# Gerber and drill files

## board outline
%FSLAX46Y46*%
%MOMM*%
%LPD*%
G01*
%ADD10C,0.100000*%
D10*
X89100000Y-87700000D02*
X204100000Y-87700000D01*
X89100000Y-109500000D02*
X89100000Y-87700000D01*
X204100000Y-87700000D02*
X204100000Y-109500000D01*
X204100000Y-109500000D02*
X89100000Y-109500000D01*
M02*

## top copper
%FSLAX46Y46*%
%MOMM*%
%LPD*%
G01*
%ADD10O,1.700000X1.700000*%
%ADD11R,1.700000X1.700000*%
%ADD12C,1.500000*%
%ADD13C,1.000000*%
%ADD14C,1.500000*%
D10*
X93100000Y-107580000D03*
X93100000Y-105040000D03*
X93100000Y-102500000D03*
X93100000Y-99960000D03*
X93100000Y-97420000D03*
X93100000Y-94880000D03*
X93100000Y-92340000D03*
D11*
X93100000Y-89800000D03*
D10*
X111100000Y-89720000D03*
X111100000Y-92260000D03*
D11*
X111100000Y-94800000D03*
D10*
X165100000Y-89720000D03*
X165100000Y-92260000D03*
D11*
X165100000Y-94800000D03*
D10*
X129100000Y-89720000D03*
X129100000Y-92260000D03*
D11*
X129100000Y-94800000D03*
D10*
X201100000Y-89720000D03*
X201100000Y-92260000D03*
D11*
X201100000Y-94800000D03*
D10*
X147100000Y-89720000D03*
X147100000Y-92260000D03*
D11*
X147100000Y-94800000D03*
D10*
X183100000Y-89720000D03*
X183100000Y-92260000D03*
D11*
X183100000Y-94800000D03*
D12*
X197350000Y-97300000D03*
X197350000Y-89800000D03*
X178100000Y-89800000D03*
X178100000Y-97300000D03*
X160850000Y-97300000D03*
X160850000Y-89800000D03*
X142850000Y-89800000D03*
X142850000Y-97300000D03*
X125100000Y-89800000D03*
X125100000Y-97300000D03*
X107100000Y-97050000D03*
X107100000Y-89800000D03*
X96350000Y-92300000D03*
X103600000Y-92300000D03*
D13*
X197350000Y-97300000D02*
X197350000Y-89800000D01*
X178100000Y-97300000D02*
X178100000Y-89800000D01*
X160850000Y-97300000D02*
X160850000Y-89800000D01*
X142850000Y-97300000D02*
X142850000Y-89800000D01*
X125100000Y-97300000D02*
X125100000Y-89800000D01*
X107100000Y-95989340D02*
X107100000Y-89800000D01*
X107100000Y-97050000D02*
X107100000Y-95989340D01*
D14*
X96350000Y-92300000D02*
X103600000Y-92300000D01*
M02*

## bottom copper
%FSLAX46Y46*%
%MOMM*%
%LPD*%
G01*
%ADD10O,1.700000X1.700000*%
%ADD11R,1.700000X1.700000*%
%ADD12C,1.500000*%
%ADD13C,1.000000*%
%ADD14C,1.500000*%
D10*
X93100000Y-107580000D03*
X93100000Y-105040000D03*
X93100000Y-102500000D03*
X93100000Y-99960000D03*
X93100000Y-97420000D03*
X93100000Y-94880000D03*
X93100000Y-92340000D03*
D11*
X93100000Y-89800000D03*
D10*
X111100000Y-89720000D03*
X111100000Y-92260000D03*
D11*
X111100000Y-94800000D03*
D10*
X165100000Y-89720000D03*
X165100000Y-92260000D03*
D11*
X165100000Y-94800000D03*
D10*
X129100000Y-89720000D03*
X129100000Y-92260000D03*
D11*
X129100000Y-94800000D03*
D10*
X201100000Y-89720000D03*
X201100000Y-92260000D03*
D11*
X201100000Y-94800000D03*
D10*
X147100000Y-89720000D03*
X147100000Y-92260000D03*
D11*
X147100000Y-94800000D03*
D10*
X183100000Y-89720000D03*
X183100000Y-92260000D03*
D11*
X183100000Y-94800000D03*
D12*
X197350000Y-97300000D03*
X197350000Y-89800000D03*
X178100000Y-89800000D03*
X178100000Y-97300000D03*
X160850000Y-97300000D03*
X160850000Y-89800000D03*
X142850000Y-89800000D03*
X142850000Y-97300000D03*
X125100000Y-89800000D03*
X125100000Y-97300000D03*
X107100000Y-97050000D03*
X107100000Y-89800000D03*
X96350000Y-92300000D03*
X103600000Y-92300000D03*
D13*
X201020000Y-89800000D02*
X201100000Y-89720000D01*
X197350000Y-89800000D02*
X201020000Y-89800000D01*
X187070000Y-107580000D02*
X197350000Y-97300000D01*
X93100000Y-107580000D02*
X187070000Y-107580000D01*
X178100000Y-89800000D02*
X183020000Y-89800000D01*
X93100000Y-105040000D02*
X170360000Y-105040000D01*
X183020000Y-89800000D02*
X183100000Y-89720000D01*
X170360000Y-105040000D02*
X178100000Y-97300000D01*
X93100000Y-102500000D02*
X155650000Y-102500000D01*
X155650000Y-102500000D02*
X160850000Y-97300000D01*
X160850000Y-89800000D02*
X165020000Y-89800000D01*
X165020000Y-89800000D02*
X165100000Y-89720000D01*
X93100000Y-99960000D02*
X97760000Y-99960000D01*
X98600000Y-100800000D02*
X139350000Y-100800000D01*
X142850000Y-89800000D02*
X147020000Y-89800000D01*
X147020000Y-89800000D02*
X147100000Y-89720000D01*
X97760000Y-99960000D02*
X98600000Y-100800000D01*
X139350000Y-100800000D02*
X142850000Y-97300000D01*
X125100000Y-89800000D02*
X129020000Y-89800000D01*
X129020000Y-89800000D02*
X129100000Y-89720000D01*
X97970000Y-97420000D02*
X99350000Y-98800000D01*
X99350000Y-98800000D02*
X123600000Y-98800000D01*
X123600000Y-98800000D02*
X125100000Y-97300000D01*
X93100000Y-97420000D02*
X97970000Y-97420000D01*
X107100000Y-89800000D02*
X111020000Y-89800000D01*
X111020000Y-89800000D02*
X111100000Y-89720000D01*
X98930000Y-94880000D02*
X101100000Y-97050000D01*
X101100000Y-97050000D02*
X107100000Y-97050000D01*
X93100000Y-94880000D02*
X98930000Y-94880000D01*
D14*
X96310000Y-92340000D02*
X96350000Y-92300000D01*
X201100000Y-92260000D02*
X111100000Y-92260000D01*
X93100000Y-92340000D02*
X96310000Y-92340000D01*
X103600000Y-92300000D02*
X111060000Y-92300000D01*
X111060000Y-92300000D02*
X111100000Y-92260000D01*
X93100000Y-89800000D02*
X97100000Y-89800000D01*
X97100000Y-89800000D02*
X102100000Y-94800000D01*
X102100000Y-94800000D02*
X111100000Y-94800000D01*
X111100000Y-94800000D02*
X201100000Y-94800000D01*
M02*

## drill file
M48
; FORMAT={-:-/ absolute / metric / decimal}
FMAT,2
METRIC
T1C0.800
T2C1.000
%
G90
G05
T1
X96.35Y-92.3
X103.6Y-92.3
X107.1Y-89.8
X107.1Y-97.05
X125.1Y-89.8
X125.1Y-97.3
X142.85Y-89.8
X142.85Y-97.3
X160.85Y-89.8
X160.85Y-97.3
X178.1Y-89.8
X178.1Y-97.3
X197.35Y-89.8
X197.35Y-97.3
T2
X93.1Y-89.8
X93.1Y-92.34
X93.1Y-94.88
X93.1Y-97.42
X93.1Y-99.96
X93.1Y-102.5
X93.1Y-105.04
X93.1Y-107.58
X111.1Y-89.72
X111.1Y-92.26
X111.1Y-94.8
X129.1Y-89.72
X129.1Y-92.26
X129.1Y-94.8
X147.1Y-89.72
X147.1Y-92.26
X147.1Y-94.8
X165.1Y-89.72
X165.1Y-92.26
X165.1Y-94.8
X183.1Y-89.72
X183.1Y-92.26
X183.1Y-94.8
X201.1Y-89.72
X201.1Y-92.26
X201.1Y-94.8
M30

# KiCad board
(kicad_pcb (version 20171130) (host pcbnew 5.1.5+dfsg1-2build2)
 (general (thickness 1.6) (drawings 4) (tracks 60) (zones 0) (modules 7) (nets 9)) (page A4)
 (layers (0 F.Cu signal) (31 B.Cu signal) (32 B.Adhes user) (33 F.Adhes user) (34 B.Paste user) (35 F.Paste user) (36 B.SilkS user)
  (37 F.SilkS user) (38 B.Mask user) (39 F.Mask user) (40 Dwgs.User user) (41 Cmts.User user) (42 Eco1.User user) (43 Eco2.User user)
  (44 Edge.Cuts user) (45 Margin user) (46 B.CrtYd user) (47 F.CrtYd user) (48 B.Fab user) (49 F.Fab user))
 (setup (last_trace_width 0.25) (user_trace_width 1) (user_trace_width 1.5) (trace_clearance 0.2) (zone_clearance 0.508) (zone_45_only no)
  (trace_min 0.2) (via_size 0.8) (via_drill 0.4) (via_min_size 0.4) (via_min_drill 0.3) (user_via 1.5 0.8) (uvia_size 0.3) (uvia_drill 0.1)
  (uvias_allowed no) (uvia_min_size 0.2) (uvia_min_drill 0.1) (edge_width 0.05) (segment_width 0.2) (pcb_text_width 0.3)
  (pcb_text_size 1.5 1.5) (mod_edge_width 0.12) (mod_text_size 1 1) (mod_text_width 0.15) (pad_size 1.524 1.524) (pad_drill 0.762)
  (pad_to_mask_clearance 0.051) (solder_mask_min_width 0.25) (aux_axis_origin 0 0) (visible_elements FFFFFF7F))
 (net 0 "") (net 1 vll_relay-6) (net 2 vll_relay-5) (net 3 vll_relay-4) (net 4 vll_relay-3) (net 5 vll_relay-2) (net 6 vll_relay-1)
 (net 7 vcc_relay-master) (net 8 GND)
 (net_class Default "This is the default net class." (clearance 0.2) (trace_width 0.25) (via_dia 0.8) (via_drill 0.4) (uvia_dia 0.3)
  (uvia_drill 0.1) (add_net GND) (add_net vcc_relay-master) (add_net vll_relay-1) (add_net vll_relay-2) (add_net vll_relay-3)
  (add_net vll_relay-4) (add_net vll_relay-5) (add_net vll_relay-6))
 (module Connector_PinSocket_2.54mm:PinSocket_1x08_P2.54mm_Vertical (layer F.Cu) (at 93.1 89.8)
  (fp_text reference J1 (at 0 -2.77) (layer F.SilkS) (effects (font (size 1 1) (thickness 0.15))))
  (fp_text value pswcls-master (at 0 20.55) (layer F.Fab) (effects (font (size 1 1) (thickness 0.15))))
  (pad 8 thru_hole oval (at 0 17.78) (size 1.7 1.7) (drill 1) (layers *.Cu *.Mask) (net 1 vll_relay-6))
  (pad 7 thru_hole oval (at 0 15.24) (size 1.7 1.7) (drill 1) (layers *.Cu *.Mask) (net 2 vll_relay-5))
  (pad 6 thru_hole oval (at 0 12.7) (size 1.7 1.7) (drill 1) (layers *.Cu *.Mask) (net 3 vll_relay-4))
  (pad 5 thru_hole oval (at 0 10.16) (size 1.7 1.7) (drill 1) (layers *.Cu *.Mask) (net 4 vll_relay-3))
  (pad 4 thru_hole oval (at 0 7.62) (size 1.7 1.7) (drill 1) (layers *.Cu *.Mask) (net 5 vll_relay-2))
  (pad 3 thru_hole oval (at 0 5.08) (size 1.7 1.7) (drill 1) (layers *.Cu *.Mask) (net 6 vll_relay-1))
  (pad 2 thru_hole oval (at 0 2.54) (size 1.7 1.7) (drill 1) (layers *.Cu *.Mask) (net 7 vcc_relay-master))
  (pad 1 thru_hole rect (at 0 0) (size 1.7 1.7) (drill 1) (layers *.Cu *.Mask) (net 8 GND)))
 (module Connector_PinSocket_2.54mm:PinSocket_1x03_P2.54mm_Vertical (layer F.Cu) (at 111.1 94.8 180)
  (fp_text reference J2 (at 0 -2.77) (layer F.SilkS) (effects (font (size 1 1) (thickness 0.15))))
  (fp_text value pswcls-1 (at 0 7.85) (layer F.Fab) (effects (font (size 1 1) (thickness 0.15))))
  (pad 3 thru_hole oval (at 0 5.08 180) (size 1.7 1.7) (drill 1) (layers *.Cu *.Mask) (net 6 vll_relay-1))
  (pad 2 thru_hole oval (at 0 2.54 180) (size 1.7 1.7) (drill 1) (layers *.Cu *.Mask) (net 7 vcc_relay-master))
  (pad 1 thru_hole rect (at 0 0 180) (size 1.7 1.7) (drill 1) (layers *.Cu *.Mask) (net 8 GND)))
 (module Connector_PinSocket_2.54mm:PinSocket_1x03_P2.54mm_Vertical (layer F.Cu) (at 165.1 94.8 180)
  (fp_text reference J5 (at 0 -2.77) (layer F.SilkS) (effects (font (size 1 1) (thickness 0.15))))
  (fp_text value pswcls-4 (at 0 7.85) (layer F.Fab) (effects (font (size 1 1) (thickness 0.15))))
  (pad 3 thru_hole oval (at 0 5.08 180) (size 1.7 1.7) (drill 1) (layers *.Cu *.Mask) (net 3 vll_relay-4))
  (pad 2 thru_hole oval (at 0 2.54 180) (size 1.7 1.7) (drill 1) (layers *.Cu *.Mask) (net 7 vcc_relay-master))
  (pad 1 thru_hole rect (at 0 0 180) (size 1.7 1.7) (drill 1) (layers *.Cu *.Mask) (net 8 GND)))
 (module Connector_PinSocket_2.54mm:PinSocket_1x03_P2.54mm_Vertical (layer F.Cu) (at 129.1 94.8 180)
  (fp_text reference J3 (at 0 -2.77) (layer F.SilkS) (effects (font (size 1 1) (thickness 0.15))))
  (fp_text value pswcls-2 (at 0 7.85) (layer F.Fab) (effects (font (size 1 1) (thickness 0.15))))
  (pad 3 thru_hole oval (at 0 5.08 180) (size 1.7 1.7) (drill 1) (layers *.Cu *.Mask) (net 5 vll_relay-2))
  (pad 2 thru_hole oval (at 0 2.54 180) (size 1.7 1.7) (drill 1) (layers *.Cu *.Mask) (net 7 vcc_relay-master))
  (pad 1 thru_hole rect (at 0 0 180) (size 1.7 1.7) (drill 1) (layers *.Cu *.Mask) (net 8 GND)))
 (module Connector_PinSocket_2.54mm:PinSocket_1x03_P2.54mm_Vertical (layer F.Cu) (at 201.1 94.8 180)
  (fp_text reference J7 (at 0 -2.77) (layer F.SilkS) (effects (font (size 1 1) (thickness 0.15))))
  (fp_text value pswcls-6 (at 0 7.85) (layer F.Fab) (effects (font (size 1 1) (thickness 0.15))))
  (pad 3 thru_hole oval (at 0 5.08 180) (size 1.7 1.7) (drill 1) (layers *.Cu *.Mask) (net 1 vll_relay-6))
  (pad 2 thru_hole oval (at 0 2.54 180) (size 1.7 1.7) (drill 1) (layers *.Cu *.Mask) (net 7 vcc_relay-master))
  (pad 1 thru_hole rect (at 0 0 180) (size 1.7 1.7) (drill 1) (layers *.Cu *.Mask) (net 8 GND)))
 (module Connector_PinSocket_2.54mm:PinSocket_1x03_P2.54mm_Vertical (layer F.Cu) (at 147.1 94.8 180)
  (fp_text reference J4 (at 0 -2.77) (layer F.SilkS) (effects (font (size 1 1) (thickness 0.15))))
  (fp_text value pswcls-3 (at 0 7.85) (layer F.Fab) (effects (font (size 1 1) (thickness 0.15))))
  (pad 3 thru_hole oval (at 0 5.08 180) (size 1.7 1.7) (drill 1) (layers *.Cu *.Mask) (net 4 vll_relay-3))
  (pad 2 thru_hole oval (at 0 2.54 180) (size 1.7 1.7) (drill 1) (layers *.Cu *.Mask) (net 7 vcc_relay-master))
  (pad 1 thru_hole rect (at 0 0 180) (size 1.7 1.7) (drill 1) (layers *.Cu *.Mask) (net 8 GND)))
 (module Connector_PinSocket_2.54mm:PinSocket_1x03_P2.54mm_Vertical (layer F.Cu) (at 183.1 94.8 180)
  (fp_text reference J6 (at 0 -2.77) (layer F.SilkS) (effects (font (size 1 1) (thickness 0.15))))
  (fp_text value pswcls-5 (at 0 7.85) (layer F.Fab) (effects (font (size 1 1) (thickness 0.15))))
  (pad 3 thru_hole oval (at 0 5.08 180) (size 1.7 1.7) (drill 1) (layers *.Cu *.Mask) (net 2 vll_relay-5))
  (pad 2 thru_hole oval (at 0 2.54 180) (size 1.7 1.7) (drill 1) (layers *.Cu *.Mask) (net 7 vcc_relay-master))
  (pad 1 thru_hole rect (at 0 0 180) (size 1.7 1.7) (drill 1) (layers *.Cu *.Mask) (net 8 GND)))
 (gr_line (start 89.1 87.7) (end 204.1 87.7) (layer Edge.Cuts) (width 0.1))
 (gr_line (start 89.1 109.5) (end 89.1 87.7) (layer Edge.Cuts) (width 0.1))
 (gr_line (start 204.1 87.7) (end 204.1 109.5) (layer Edge.Cuts) (width 0.1))
 (gr_line (start 204.1 109.5) (end 89.1 109.5) (layer Edge.Cuts) (width 0.1))
 (segment (start 201.02 89.8) (end 201.1 89.72) (width 1) (layer B.Cu) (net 1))
 (via (at 197.35 97.3) (size 1.5) (drill 0.8) (layers F.Cu B.Cu) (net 1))
 (via (at 197.35 89.8) (size 1.5) (drill 0.8) (layers F.Cu B.Cu) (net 1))
 (segment (start 197.35 89.8) (end 201.02 89.8) (width 1) (layer B.Cu) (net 1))
 (segment (start 197.35 97.3) (end 197.35 89.8) (width 1) (layer F.Cu) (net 1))
 (segment (start 187.07 107.58) (end 197.35 97.3) (width 1) (layer B.Cu) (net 1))
 (segment (start 93.1 107.58) (end 187.07 107.58) (width 1) (layer B.Cu) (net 1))
 (via (at 178.1 89.8) (size 1.5) (drill 0.8) (layers F.Cu B.Cu) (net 2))
 (segment (start 178.1 89.8) (end 183.02 89.8) (width 1) (layer B.Cu) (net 2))
 (segment (start 93.1 105.04) (end 170.36 105.04) (width 1) (layer B.Cu) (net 2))
 (segment (start 178.1 97.3) (end 178.1 89.8) (width 1) (layer F.Cu) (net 2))
 (via (at 178.1 97.3) (size 1.5) (drill 0.8) (layers F.Cu B.Cu) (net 2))
 (segment (start 183.02 89.8) (end 183.1 89.72) (width 1) (layer B.Cu) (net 2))
 (segment (start 170.36 105.04) (end 178.1 97.3) (width 1) (layer B.Cu) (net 2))
 (segment (start 93.1 102.5) (end 155.65 102.5) (width 1) (layer B.Cu) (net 3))
 (segment (start 155.65 102.5) (end 160.85 97.3) (width 1) (layer B.Cu) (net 3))
 (via (at 160.85 97.3) (size 1.5) (drill 0.8) (layers F.Cu B.Cu) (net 3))
 (segment (start 160.85 89.8) (end 165.02 89.8) (width 1) (layer B.Cu) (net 3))
 (segment (start 165.02 89.8) (end 165.1 89.72) (width 1) (layer B.Cu) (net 3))
 (segment (start 160.85 97.3) (end 160.85 89.8) (width 1) (layer F.Cu) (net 3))
 (via (at 160.85 89.8) (size 1.5) (drill 0.8) (layers F.Cu B.Cu) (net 3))
 (segment (start 93.1 99.96) (end 97.76 99.96) (width 1) (layer B.Cu) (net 4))
 (segment (start 98.6 100.8) (end 139.35 100.8) (width 1) (layer B.Cu) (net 4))
 (via (at 142.85 89.8) (size 1.5) (drill 0.8) (layers F.Cu B.Cu) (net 4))
 (via (at 142.85 97.3) (size 1.5) (drill 0.8) (layers F.Cu B.Cu) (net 4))
 (segment (start 142.85 89.8) (end 147.02 89.8) (width 1) (layer B.Cu) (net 4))
 (segment (start 147.02 89.8) (end 147.1 89.72) (width 1) (layer B.Cu) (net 4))
 (segment (start 142.85 97.3) (end 142.85 89.8) (width 1) (layer F.Cu) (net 4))
 (segment (start 97.76 99.96) (end 98.6 100.8) (width 1) (layer B.Cu) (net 4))
 (segment (start 139.35 100.8) (end 142.85 97.3) (width 1) (layer B.Cu) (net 4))
 (segment (start 125.1 89.8) (end 129.02 89.8) (width 1) (layer B.Cu) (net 5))
 (segment (start 129.02 89.8) (end 129.1 89.72) (width 1) (layer B.Cu) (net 5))
 (segment (start 125.1 97.3) (end 125.1 89.8) (width 1) (layer F.Cu) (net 5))
 (via (at 125.1 89.8) (size 1.5) (drill 0.8) (layers F.Cu B.Cu) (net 5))
 (via (at 125.1 97.3) (size 1.5) (drill 0.8) (layers F.Cu B.Cu) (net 5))
 (segment (start 97.97 97.42) (end 99.35 98.8) (width 1) (layer B.Cu) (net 5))
 (segment (start 99.35 98.8) (end 123.6 98.8) (width 1) (layer B.Cu) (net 5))
 (segment (start 123.6 98.8) (end 125.1 97.3) (width 1) (layer B.Cu) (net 5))
 (segment (start 93.1 97.42) (end 97.97 97.42) (width 1) (layer B.Cu) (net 5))
 (segment (start 107.1 89.8) (end 111.02 89.8) (width 1) (layer B.Cu) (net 6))
 (segment (start 111.02 89.8) (end 111.1 89.72) (width 1) (layer B.Cu) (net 6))
 (segment (start 107.1 95.98934) (end 107.1 89.8) (width 1) (layer F.Cu) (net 6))
 (segment (start 98.93 94.88) (end 101.1 97.05) (width 1) (layer B.Cu) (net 6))
 (segment (start 101.1 97.05) (end 107.1 97.05) (width 1) (layer B.Cu) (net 6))
 (via (at 107.1 97.05) (size 1.5) (drill 0.8) (layers F.Cu B.Cu) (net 6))
 (segment (start 93.1 94.88) (end 98.93 94.88) (width 1) (layer B.Cu) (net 6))
 (via (at 107.1 89.8) (size 1.5) (drill 0.8) (layers F.Cu B.Cu) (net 6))
 (segment (start 107.1 97.05) (end 107.1 95.98934) (width 1) (layer F.Cu) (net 6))
 (segment (start 96.31 92.34) (end 96.35 92.3) (width 1.5) (layer B.Cu) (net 7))
 (via (at 96.35 92.3) (size 1.5) (drill 0.8) (layers F.Cu B.Cu) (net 7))
 (segment (start 201.1 92.26) (end 111.1 92.26) (width 1.5) (layer B.Cu) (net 7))
 (via (at 103.6 92.3) (size 1.5) (drill 0.8) (layers F.Cu B.Cu) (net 7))
 (segment (start 93.1 92.34) (end 96.31 92.34) (width 1.5) (layer B.Cu) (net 7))
 (segment (start 103.6 92.3) (end 111.06 92.3) (width 1.5) (layer B.Cu) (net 7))
 (segment (start 111.06 92.3) (end 111.1 92.26) (width 1.5) (layer B.Cu) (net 7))
 (segment (start 96.35 92.3) (end 103.6 92.3) (width 1.5) (layer F.Cu) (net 7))
 (segment (start 93.1 89.8) (end 97.1 89.8) (width 1.5) (layer B.Cu) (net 8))
 (segment (start 97.1 89.8) (end 102.1 94.8) (width 1.5) (layer B.Cu) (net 8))
 (segment (start 102.1 94.8) (end 111.1 94.8) (width 1.5) (layer B.Cu) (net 8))
 (segment (start 111.1 94.8) (end 201.1 94.8) (width 1.5) (layer B.Cu) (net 8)))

